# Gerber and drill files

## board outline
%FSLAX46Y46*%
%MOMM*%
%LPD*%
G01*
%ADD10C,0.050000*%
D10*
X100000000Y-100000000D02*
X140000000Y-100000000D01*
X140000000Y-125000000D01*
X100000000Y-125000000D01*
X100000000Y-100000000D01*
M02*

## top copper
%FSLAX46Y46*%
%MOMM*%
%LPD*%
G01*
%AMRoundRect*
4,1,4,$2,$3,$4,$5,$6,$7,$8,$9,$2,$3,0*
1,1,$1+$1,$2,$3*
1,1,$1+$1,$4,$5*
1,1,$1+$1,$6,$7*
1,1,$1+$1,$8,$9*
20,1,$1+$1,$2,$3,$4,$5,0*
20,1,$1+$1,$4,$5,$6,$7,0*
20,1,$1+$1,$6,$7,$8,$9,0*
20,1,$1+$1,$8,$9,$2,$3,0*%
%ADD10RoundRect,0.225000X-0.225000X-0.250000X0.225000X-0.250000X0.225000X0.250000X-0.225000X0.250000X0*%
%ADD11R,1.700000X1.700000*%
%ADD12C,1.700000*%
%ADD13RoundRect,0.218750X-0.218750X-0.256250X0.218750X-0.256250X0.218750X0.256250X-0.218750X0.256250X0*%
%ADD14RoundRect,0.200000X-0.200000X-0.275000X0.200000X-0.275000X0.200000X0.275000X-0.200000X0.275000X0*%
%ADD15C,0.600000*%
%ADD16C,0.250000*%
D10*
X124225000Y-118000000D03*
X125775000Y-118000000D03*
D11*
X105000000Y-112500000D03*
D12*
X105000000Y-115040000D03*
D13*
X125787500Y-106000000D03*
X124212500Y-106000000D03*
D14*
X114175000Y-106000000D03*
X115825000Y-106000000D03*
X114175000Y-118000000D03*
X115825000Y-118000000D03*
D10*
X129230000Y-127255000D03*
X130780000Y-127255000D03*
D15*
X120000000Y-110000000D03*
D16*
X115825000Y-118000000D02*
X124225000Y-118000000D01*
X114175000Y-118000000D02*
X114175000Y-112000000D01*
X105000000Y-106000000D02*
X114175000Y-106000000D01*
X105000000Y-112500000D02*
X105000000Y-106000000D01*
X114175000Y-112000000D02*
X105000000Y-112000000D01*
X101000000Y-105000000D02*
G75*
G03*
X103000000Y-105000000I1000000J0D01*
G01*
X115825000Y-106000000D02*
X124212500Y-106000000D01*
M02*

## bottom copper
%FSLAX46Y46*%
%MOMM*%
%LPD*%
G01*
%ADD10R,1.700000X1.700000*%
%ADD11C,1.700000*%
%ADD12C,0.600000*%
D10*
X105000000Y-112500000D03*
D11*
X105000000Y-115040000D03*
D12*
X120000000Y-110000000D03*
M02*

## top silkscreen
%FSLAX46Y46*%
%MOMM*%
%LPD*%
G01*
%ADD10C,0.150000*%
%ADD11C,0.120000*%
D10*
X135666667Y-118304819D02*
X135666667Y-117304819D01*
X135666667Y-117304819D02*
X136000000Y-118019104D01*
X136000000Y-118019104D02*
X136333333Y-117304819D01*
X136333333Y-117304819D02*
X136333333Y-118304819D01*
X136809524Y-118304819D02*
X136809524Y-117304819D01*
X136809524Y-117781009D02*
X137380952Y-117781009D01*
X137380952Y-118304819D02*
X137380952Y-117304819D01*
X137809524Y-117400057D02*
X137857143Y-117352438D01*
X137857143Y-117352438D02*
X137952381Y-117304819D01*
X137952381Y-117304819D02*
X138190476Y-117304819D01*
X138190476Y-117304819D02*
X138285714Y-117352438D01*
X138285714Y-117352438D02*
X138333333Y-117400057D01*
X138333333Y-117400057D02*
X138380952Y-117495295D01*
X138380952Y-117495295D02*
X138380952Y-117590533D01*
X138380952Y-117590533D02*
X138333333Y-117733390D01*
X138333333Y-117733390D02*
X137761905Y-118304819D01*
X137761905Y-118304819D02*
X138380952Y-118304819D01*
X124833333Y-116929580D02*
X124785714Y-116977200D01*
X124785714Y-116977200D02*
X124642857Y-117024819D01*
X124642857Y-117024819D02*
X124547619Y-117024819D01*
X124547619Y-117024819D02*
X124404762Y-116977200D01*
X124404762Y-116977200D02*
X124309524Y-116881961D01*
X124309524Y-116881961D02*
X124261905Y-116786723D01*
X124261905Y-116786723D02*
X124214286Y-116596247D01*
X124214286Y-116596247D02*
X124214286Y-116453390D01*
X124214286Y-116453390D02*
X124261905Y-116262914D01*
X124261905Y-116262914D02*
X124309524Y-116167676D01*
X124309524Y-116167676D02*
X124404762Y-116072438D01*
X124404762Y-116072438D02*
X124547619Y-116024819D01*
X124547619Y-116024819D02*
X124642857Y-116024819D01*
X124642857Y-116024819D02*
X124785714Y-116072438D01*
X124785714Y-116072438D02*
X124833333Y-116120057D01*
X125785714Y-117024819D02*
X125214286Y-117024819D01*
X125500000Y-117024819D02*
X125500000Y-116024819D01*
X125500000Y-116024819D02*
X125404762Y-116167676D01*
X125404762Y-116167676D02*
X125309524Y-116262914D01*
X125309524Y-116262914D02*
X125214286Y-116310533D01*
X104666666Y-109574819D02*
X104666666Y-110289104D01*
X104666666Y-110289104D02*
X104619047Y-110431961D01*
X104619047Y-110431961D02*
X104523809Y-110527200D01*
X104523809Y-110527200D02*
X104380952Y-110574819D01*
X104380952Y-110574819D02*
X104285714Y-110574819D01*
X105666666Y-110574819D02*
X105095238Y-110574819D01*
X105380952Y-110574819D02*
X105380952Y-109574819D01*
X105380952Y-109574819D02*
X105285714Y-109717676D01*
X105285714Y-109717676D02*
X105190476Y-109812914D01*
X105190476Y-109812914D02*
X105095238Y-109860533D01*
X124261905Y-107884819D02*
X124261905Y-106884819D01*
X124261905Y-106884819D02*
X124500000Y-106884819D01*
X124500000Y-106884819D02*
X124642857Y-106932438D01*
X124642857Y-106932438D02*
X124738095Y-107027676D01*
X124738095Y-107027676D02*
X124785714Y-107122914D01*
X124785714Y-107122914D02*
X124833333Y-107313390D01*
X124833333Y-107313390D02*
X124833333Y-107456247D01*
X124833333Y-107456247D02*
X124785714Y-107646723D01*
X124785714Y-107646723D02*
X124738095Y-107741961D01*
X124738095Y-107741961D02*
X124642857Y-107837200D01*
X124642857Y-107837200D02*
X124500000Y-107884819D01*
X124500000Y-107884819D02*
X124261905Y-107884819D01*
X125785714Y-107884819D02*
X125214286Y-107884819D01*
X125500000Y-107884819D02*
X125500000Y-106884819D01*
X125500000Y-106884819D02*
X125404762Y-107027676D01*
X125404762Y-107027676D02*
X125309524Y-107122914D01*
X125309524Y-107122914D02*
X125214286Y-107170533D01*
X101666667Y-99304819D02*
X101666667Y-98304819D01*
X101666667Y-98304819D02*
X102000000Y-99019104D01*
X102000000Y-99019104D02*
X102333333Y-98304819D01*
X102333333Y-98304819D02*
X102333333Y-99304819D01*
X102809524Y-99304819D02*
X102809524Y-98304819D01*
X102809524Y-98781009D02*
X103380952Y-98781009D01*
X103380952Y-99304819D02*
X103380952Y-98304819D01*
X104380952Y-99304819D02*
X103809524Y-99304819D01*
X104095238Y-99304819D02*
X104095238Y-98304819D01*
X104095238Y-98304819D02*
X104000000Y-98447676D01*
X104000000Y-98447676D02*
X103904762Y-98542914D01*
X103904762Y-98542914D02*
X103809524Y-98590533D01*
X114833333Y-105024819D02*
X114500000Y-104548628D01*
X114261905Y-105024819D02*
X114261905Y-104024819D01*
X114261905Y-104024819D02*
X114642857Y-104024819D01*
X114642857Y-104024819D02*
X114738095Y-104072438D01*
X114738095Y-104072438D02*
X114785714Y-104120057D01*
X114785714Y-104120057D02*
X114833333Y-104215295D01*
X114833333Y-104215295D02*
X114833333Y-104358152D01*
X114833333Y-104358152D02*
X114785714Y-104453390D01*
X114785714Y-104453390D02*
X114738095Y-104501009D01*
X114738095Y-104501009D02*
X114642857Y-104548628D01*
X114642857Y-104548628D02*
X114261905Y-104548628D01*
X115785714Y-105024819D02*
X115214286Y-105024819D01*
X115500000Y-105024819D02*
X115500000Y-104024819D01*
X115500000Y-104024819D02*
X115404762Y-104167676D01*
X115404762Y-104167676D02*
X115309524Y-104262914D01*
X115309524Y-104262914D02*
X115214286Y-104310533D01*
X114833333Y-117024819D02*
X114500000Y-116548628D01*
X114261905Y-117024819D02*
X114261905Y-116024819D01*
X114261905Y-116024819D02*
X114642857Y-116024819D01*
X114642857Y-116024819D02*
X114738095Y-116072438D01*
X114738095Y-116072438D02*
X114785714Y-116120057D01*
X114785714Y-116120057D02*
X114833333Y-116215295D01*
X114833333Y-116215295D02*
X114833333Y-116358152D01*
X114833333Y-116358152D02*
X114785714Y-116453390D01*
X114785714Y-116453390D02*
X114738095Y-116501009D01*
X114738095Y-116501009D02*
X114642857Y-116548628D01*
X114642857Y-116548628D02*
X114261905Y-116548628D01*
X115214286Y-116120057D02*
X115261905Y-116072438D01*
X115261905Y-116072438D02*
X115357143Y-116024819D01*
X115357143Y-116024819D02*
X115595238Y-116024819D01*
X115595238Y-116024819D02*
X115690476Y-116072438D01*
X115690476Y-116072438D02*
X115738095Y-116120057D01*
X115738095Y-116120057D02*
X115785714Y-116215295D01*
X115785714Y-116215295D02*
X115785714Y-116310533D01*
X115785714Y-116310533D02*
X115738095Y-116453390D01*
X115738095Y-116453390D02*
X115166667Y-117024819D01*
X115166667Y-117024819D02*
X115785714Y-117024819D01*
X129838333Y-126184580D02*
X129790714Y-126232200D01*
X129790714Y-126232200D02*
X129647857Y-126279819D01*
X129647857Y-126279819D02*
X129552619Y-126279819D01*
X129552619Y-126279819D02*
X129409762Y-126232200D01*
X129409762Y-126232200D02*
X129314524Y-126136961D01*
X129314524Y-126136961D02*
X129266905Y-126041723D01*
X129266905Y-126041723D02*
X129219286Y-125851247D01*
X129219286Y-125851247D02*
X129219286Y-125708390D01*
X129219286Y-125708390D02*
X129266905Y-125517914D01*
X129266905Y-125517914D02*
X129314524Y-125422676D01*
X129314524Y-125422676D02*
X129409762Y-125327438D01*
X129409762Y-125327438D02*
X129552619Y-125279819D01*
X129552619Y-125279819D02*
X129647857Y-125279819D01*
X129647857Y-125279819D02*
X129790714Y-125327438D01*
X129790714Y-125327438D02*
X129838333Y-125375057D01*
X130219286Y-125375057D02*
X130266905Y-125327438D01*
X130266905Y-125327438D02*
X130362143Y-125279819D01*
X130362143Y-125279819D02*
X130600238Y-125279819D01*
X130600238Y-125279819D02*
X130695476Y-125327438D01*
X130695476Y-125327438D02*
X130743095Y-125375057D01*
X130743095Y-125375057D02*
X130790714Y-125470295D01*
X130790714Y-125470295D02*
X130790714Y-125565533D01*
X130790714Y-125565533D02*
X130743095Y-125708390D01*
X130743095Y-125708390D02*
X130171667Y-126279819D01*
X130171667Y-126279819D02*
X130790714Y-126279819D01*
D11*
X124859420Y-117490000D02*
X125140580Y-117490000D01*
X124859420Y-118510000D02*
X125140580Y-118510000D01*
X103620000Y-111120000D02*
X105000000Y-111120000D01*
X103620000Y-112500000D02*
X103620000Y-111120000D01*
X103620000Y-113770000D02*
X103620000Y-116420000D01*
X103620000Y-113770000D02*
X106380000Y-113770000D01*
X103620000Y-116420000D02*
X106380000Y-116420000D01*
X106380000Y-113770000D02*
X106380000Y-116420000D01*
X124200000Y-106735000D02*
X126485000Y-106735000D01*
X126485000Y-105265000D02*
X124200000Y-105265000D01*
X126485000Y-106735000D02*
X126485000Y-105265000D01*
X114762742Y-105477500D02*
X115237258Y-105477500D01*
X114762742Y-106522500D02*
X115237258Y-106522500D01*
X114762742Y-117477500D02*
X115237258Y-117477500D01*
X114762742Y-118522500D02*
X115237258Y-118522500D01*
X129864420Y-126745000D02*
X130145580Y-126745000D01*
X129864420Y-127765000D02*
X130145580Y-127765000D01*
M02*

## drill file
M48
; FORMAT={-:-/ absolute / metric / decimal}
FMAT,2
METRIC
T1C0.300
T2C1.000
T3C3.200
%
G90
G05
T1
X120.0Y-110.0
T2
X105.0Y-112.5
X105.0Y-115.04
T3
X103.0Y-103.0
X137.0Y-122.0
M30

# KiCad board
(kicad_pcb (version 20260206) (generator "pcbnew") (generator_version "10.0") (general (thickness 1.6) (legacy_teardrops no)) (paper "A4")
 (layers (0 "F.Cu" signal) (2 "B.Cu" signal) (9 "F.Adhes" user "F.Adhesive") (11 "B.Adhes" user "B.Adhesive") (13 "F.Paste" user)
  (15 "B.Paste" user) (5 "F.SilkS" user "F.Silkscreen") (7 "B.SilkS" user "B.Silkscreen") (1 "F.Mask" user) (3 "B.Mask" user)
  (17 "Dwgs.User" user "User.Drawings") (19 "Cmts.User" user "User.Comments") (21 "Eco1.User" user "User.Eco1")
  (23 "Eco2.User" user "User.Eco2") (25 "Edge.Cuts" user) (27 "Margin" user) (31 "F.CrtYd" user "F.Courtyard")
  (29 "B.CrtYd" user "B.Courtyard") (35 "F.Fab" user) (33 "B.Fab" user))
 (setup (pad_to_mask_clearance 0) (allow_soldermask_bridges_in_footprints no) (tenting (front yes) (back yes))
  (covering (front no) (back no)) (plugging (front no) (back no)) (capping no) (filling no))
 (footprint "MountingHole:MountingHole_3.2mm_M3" (layer "F.Cu") (at 137 122)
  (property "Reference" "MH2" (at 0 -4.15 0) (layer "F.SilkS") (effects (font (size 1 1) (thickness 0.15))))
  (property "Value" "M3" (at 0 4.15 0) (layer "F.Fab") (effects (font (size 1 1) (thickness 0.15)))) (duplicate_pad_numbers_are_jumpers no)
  (pad "" np_thru_hole circle (at 0 0) (size 3.2 3.2) (drill 3.2) (layers "*.Cu" "*.Mask")))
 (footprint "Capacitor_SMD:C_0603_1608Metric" (layer "F.Cu") (at 125 118)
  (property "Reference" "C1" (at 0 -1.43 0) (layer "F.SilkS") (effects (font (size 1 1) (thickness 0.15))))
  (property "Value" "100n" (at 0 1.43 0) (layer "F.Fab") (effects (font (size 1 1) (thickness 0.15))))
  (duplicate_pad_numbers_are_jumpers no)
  (fp_line (start -0.14058 -0.51) (end 0.14058 -0.51) (stroke (width 0.12) (type solid)) (layer "F.SilkS"))
  (fp_line (start -0.14058 0.51) (end 0.14058 0.51) (stroke (width 0.12) (type solid)) (layer "F.SilkS"))
  (pad "1" smd roundrect (at -0.775 0) (size 0.9 0.95) (layers "F.Cu" "F.Mask" "F.Paste") (roundrect_rratio 0.25) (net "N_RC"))
  (pad "2" smd roundrect (at 0.775 0) (size 0.9 0.95) (layers "F.Cu" "F.Mask" "F.Paste") (roundrect_rratio 0.25) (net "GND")))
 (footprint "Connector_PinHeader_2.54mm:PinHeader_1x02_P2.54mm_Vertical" (layer "F.Cu") (at 105 112.5)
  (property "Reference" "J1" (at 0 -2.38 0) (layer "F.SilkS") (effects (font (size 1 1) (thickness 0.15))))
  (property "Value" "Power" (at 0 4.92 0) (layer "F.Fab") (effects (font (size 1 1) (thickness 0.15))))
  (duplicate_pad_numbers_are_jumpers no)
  (fp_line (start -1.38 -1.38) (end 0 -1.38) (stroke (width 0.12) (type solid)) (layer "F.SilkS"))
  (fp_line (start -1.38 0) (end -1.38 -1.38) (stroke (width 0.12) (type solid)) (layer "F.SilkS"))
  (fp_line (start -1.38 1.27) (end -1.38 3.92) (stroke (width 0.12) (type solid)) (layer "F.SilkS"))
  (fp_line (start -1.38 1.27) (end 1.38 1.27) (stroke (width 0.12) (type solid)) (layer "F.SilkS"))
  (fp_line (start -1.38 3.92) (end 1.38 3.92) (stroke (width 0.12) (type solid)) (layer "F.SilkS"))
  (fp_line (start 1.38 1.27) (end 1.38 3.92) (stroke (width 0.12) (type solid)) (layer "F.SilkS"))
  (pad "1" thru_hole rect (at 0 0) (size 1.7 1.7) (drill 1) (layers "*.Cu" "*.Mask") (remove_unused_layers no) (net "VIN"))
  (pad "2" thru_hole circle (at 0 2.54) (size 1.7 1.7) (drill 1) (layers "*.Cu" "*.Mask") (remove_unused_layers no) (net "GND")))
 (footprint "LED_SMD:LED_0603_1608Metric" (layer "F.Cu") (at 125 106 180)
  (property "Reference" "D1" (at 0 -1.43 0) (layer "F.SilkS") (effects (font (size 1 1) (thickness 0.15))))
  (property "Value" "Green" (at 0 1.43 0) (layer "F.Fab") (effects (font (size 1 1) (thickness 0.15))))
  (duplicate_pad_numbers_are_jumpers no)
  (fp_line (start 0.8 -0.735) (end -1.485 -0.735) (stroke (width 0.12) (type solid)) (layer "F.SilkS"))
  (fp_line (start -1.485 0.735) (end 0.8 0.735) (stroke (width 0.12) (type solid)) (layer "F.SilkS"))
  (fp_line (start -1.485 -0.735) (end -1.485 0.735) (stroke (width 0.12) (type solid)) (layer "F.SilkS"))
  (pad "1" smd roundrect (at -0.7875 0) (size 0.875 0.95) (layers "F.Cu" "F.Mask" "F.Paste") (roundrect_rratio 0.25) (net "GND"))
  (pad "2" smd roundrect (at 0.7875 0) (size 0.875 0.95) (layers "F.Cu" "F.Mask" "F.Paste") (roundrect_rratio 0.25) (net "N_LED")))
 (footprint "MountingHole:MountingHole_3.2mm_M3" (layer "F.Cu") (at 103 103)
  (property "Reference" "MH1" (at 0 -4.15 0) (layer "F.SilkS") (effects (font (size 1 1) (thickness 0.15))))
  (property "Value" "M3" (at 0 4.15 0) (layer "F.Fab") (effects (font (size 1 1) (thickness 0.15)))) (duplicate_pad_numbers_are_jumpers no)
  (pad "" np_thru_hole circle (at 0 0) (size 3.2 3.2) (drill 3.2) (layers "*.Cu" "*.Mask")))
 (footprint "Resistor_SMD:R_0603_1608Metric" (layer "F.Cu") (at 115 106)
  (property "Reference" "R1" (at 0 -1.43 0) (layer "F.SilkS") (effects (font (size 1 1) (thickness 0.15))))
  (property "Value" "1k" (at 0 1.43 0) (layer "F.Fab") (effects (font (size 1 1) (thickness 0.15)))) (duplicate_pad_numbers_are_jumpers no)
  (fp_line (start -0.237258 -0.5225) (end 0.237258 -0.5225) (stroke (width 0.12) (type solid)) (layer "F.SilkS"))
  (fp_line (start -0.237258 0.5225) (end 0.237258 0.5225) (stroke (width 0.12) (type solid)) (layer "F.SilkS"))
  (pad "1" smd roundrect (at -0.825 0) (size 0.8 0.95) (layers "F.Cu" "F.Mask" "F.Paste") (roundrect_rratio 0.25) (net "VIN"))
  (pad "2" smd roundrect (at 0.825 0) (size 0.8 0.95) (layers "F.Cu" "F.Mask" "F.Paste") (roundrect_rratio 0.25) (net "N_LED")))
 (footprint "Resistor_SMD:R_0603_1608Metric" (layer "F.Cu") (at 115 118)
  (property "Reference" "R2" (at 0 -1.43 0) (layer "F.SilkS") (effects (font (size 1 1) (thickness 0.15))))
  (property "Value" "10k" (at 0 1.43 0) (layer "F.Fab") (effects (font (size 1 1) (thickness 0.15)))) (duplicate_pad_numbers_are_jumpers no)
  (fp_line (start -0.237258 -0.5225) (end 0.237258 -0.5225) (stroke (width 0.12) (type solid)) (layer "F.SilkS"))
  (fp_line (start -0.237258 0.5225) (end 0.237258 0.5225) (stroke (width 0.12) (type solid)) (layer "F.SilkS"))
  (pad "1" smd roundrect (at -0.825 0) (size 0.8 0.95) (layers "F.Cu" "F.Mask" "F.Paste") (roundrect_rratio 0.25) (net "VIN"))
  (pad "2" smd roundrect (at 0.825 0) (size 0.8 0.95) (layers "F.Cu" "F.Mask" "F.Paste") (roundrect_rratio 0.25) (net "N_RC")))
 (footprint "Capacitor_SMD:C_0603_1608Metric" (layer "F.Cu") (at 130.005 127.255)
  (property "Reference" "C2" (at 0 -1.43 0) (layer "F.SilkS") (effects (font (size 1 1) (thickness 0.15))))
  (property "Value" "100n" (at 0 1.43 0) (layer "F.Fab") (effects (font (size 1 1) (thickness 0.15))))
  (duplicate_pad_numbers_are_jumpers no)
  (fp_line (start -0.14058 -0.51) (end 0.14058 -0.51) (stroke (width 0.12) (type solid)) (layer "F.SilkS"))
  (fp_line (start -0.14058 0.51) (end 0.14058 0.51) (stroke (width 0.12) (type solid)) (layer "F.SilkS"))
  (pad "1" smd roundrect (at -0.775 0) (size 0.9 0.95) (layers "F.Cu" "F.Mask" "F.Paste") (roundrect_rratio 0.25) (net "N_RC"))
  (pad "2" smd roundrect (at 0.775 0) (size 0.9 0.95) (layers "F.Cu" "F.Mask" "F.Paste") (roundrect_rratio 0.25) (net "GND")))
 (gr_rect (start 100 100) (end 140 125) (stroke (width 0.05) (type default)) (fill no) (layer "Edge.Cuts"))
 (segment (start 115.825 118) (end 124.225 118) (width 0.25) (layer "F.Cu") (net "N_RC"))
 (segment (start 114.175 118) (end 114.175 112) (width 0.25) (layer "F.Cu") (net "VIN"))
 (segment (start 105 106) (end 114.175 106) (width 0.25) (layer "F.Cu") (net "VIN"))
 (segment (start 105 112.5) (end 105 106) (width 0.25) (layer "F.Cu") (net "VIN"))
 (segment (start 114.175 112) (end 105 112) (width 0.25) (layer "F.Cu") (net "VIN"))
 (via (at 120 110) (size 0.6) (drill 0.3) (layers "F.Cu" "B.Cu") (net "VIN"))
 (arc (start 101 105) (mid 102 106) (end 103 105) (width 0.25) (layer "F.Cu") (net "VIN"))
 (segment (start 115.825 106) (end 124.2125 106) (width 0.25) (layer "F.Cu") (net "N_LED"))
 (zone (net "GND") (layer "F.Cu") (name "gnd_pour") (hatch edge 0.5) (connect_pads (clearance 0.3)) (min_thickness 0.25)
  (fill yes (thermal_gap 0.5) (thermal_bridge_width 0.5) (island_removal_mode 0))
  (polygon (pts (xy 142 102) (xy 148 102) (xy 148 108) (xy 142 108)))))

